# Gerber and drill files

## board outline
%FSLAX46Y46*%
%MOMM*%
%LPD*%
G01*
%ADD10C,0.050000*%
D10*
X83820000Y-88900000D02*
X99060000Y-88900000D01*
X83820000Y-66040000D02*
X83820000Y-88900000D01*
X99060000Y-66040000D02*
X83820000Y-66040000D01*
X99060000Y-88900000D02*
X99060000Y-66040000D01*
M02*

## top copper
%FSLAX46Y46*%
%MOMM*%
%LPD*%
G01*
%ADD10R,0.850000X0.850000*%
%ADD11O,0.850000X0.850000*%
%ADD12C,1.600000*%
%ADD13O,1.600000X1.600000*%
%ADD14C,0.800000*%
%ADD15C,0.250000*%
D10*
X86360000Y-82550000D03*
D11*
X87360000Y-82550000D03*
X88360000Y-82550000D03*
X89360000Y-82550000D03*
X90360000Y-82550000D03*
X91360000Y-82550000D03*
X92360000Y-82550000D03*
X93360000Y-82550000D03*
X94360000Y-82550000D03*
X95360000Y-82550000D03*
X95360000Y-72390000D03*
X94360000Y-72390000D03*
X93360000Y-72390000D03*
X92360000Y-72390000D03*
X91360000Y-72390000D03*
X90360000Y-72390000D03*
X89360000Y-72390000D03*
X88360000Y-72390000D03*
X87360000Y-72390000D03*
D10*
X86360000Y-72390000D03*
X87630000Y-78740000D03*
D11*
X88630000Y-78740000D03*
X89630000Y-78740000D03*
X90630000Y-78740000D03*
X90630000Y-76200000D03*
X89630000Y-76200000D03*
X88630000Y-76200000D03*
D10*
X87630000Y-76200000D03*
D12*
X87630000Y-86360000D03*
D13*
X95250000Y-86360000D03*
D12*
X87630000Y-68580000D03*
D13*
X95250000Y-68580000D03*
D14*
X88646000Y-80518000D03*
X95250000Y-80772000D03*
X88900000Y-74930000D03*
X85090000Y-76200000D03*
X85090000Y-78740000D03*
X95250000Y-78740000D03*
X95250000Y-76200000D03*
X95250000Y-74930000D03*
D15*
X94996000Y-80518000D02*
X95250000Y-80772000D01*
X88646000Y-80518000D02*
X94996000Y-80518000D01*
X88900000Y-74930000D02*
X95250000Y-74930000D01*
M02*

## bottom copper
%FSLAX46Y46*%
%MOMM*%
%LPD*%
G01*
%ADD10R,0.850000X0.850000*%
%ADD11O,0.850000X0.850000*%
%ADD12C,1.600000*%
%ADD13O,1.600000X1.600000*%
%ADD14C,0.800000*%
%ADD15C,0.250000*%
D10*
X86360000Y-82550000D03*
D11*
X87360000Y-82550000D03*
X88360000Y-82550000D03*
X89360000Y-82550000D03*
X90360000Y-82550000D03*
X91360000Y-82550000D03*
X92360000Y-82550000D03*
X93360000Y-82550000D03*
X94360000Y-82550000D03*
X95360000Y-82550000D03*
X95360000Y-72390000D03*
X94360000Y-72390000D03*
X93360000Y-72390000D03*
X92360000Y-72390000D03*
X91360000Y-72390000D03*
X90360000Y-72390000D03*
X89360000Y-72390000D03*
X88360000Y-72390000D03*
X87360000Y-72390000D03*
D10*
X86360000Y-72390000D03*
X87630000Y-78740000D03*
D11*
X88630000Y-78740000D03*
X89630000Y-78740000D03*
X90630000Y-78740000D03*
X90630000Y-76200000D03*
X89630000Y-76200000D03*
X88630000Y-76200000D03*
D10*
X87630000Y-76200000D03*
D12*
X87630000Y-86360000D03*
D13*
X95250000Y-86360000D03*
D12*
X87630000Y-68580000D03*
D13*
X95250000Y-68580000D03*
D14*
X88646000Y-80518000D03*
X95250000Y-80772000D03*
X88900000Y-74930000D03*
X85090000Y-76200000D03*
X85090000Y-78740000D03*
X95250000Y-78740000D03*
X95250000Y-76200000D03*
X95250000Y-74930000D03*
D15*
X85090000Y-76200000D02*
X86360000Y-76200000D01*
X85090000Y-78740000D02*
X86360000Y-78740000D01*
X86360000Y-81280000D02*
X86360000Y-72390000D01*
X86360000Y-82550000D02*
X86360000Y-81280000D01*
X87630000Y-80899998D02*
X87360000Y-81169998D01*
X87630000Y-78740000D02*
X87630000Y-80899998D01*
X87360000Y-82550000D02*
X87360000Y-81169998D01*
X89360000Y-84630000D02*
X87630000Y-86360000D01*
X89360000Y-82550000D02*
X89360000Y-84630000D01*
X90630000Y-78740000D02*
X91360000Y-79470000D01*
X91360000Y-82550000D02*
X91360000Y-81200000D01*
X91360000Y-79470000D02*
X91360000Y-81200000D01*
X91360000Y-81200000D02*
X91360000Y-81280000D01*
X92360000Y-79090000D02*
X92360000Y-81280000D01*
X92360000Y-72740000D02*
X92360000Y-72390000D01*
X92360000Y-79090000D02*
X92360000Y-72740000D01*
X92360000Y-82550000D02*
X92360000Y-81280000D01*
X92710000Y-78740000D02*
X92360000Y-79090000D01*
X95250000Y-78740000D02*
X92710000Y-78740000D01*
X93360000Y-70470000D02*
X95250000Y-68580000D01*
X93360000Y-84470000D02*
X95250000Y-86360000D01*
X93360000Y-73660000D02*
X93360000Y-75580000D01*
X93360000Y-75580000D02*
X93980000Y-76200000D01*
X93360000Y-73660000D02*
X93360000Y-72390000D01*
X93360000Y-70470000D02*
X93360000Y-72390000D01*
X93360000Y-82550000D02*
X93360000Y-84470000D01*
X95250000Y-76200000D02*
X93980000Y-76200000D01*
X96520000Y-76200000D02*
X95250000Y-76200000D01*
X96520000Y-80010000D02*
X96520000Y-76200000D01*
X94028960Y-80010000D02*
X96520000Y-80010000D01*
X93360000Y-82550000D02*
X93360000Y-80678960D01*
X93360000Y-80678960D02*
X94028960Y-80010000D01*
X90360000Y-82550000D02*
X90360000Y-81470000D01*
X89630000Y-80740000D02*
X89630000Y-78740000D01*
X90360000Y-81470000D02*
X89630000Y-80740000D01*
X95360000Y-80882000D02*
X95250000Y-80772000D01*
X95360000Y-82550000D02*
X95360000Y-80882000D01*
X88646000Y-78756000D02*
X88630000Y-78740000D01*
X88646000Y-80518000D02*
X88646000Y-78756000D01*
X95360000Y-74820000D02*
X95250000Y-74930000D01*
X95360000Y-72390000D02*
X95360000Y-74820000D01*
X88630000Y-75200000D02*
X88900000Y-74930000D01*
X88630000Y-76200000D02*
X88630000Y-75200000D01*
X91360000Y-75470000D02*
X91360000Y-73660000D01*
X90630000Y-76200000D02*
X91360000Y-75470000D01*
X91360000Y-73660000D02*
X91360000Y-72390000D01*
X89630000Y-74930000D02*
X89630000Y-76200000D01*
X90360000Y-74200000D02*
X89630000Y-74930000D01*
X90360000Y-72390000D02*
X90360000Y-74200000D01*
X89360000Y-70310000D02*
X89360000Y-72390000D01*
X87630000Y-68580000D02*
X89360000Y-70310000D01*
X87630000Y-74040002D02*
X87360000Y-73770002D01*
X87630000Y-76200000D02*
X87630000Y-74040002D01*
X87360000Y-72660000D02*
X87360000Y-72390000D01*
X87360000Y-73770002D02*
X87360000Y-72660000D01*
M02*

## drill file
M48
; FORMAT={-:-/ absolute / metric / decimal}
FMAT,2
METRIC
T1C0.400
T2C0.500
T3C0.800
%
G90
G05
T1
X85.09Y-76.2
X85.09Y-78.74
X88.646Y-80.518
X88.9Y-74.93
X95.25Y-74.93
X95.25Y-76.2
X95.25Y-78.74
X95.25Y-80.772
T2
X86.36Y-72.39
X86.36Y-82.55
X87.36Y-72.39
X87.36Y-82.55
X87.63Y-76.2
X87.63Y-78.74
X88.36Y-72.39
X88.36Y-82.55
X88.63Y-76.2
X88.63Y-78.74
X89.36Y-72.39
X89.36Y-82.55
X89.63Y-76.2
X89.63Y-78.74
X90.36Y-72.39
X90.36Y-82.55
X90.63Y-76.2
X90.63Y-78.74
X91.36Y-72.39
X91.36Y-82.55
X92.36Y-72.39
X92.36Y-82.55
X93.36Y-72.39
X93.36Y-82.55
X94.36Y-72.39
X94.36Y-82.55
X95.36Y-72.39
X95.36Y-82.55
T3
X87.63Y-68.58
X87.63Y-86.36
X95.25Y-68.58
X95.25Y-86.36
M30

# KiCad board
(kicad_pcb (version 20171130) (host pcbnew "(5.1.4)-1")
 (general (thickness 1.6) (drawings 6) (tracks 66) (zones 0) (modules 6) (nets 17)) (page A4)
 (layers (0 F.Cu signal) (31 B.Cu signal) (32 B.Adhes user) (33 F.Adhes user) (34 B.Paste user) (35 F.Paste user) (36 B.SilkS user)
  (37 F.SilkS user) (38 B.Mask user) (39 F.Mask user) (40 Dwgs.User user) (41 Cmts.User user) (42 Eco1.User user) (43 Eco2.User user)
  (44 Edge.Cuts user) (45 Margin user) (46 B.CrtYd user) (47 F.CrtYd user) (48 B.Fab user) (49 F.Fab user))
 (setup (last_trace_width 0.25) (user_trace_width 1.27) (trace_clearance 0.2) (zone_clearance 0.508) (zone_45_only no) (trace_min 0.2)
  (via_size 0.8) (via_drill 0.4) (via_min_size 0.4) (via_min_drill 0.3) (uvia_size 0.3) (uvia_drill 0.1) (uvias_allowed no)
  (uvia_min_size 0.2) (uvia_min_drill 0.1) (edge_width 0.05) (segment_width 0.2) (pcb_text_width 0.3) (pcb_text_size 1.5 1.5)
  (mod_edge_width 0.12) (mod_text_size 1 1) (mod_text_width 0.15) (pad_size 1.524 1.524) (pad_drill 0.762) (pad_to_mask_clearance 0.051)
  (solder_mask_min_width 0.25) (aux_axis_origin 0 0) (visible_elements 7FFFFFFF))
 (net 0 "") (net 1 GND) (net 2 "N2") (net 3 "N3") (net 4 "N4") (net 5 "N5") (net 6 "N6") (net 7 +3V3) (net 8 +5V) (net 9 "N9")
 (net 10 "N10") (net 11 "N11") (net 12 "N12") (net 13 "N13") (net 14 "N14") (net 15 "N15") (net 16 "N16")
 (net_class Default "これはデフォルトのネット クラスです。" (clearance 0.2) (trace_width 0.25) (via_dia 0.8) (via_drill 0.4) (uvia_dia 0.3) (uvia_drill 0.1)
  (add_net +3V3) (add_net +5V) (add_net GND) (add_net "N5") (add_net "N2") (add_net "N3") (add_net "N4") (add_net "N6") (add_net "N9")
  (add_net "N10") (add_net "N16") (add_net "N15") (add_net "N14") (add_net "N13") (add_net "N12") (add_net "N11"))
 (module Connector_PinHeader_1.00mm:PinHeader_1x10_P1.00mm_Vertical (layer F.Cu) (at 86.36 82.55 90)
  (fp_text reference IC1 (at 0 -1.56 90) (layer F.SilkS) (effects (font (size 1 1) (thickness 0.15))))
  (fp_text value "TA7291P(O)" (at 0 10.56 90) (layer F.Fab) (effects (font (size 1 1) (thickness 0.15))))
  (pad 1 thru_hole rect (at 0 0 90) (size 0.85 0.85) (drill 0.5) (layers *.Cu *.Mask) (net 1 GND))
  (pad 2 thru_hole oval (at 0 1 90) (size 0.85 0.85) (drill 0.5) (layers *.Cu *.Mask) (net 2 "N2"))
  (pad 3 thru_hole oval (at 0 2 90) (size 0.85 0.85) (drill 0.5) (layers *.Cu *.Mask) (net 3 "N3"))
  (pad 4 thru_hole oval (at 0 3 90) (size 0.85 0.85) (drill 0.5) (layers *.Cu *.Mask) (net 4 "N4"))
  (pad 5 thru_hole oval (at 0 4 90) (size 0.85 0.85) (drill 0.5) (layers *.Cu *.Mask) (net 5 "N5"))
  (pad 6 thru_hole oval (at 0 5 90) (size 0.85 0.85) (drill 0.5) (layers *.Cu *.Mask) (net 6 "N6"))
  (pad 7 thru_hole oval (at 0 6 90) (size 0.85 0.85) (drill 0.5) (layers *.Cu *.Mask) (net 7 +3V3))
  (pad 8 thru_hole oval (at 0 7 90) (size 0.85 0.85) (drill 0.5) (layers *.Cu *.Mask) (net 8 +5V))
  (pad 9 thru_hole oval (at 0 8 90) (size 0.85 0.85) (drill 0.5) (layers *.Cu *.Mask) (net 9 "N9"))
  (pad 10 thru_hole oval (at 0 9 90) (size 0.85 0.85) (drill 0.5) (layers *.Cu *.Mask) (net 5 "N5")))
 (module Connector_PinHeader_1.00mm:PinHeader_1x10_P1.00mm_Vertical (layer F.Cu) (at 86.36 72.39 90)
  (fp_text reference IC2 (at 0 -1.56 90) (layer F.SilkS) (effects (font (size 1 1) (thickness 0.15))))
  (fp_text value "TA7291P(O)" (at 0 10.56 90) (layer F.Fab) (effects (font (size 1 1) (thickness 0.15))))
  (pad 10 thru_hole oval (at 0 9 90) (size 0.85 0.85) (drill 0.5) (layers *.Cu *.Mask) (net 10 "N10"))
  (pad 9 thru_hole oval (at 0 8 90) (size 0.85 0.85) (drill 0.5) (layers *.Cu *.Mask) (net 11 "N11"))
  (pad 8 thru_hole oval (at 0 7 90) (size 0.85 0.85) (drill 0.5) (layers *.Cu *.Mask) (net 8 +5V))
  (pad 7 thru_hole oval (at 0 6 90) (size 0.85 0.85) (drill 0.5) (layers *.Cu *.Mask) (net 7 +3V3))
  (pad 6 thru_hole oval (at 0 5 90) (size 0.85 0.85) (drill 0.5) (layers *.Cu *.Mask) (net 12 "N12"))
  (pad 5 thru_hole oval (at 0 4 90) (size 0.85 0.85) (drill 0.5) (layers *.Cu *.Mask) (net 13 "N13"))
  (pad 4 thru_hole oval (at 0 3 90) (size 0.85 0.85) (drill 0.5) (layers *.Cu *.Mask) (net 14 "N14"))
  (pad 3 thru_hole oval (at 0 2 90) (size 0.85 0.85) (drill 0.5) (layers *.Cu *.Mask) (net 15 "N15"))
  (pad 2 thru_hole oval (at 0 1 90) (size 0.85 0.85) (drill 0.5) (layers *.Cu *.Mask) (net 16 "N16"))
  (pad 1 thru_hole rect (at 0 0 90) (size 0.85 0.85) (drill 0.5) (layers *.Cu *.Mask) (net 1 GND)))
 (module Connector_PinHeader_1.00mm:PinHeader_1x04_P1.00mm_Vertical (layer F.Cu) (at 87.63 78.74 90)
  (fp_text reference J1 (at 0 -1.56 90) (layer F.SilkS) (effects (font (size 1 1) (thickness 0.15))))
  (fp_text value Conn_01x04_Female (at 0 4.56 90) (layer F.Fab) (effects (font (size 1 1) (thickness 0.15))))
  (pad 1 thru_hole rect (at 0 0 90) (size 0.85 0.85) (drill 0.5) (layers *.Cu *.Mask) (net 2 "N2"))
  (pad 2 thru_hole oval (at 0 1 90) (size 0.85 0.85) (drill 0.5) (layers *.Cu *.Mask) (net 5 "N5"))
  (pad 3 thru_hole oval (at 0 2 90) (size 0.85 0.85) (drill 0.5) (layers *.Cu *.Mask) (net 5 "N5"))
  (pad 4 thru_hole oval (at 0 3 90) (size 0.85 0.85) (drill 0.5) (layers *.Cu *.Mask) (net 6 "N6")))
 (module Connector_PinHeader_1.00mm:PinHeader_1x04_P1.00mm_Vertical (layer F.Cu) (at 87.63 76.2 90)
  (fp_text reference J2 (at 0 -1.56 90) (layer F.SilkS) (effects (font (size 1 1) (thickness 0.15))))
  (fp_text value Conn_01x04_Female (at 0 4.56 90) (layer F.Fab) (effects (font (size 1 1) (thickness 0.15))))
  (pad 4 thru_hole oval (at 0 3 90) (size 0.85 0.85) (drill 0.5) (layers *.Cu *.Mask) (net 12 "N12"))
  (pad 3 thru_hole oval (at 0 2 90) (size 0.85 0.85) (drill 0.5) (layers *.Cu *.Mask) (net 13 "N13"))
  (pad 2 thru_hole oval (at 0 1 90) (size 0.85 0.85) (drill 0.5) (layers *.Cu *.Mask) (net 10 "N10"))
  (pad 1 thru_hole rect (at 0 0 90) (size 0.85 0.85) (drill 0.5) (layers *.Cu *.Mask) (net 16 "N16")))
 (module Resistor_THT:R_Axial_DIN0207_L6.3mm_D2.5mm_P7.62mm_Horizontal (layer F.Cu) (at 87.63 86.36)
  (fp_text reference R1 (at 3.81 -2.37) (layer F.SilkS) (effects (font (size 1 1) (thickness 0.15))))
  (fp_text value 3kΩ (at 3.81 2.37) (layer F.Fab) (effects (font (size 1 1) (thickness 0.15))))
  (pad 1 thru_hole circle (at 0 0) (size 1.6 1.6) (drill 0.8) (layers *.Cu *.Mask) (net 4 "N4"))
  (pad 2 thru_hole oval (at 7.62 0) (size 1.6 1.6) (drill 0.8) (layers *.Cu *.Mask) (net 8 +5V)))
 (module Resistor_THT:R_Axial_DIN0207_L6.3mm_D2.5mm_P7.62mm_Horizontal (layer F.Cu) (at 87.63 68.58)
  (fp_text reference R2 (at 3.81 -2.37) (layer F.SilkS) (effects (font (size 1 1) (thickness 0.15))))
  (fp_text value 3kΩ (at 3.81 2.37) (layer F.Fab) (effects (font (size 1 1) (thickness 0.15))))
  (pad 1 thru_hole circle (at 0 0) (size 1.6 1.6) (drill 0.8) (layers *.Cu *.Mask) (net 14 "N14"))
  (pad 2 thru_hole oval (at 7.62 0) (size 1.6 1.6) (drill 0.8) (layers *.Cu *.Mask) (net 8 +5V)))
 (gr_line (start 83.82 88.9) (end 99.06 88.9) (layer Edge.Cuts) (width 0.05))
 (gr_line (start 83.82 66.04) (end 83.82 88.9) (layer Edge.Cuts) (width 0.05))
 (gr_line (start 99.06 66.04) (end 83.82 66.04) (layer Edge.Cuts) (width 0.05))
 (gr_line (start 99.06 88.9) (end 99.06 66.04) (layer Edge.Cuts) (width 0.05))
 (via (at 88.646 80.518) (size 0.8) (drill 0.4) (layers F.Cu B.Cu) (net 5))
 (via (at 95.25 80.772) (size 0.8) (drill 0.4) (layers F.Cu B.Cu) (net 5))
 (segment (start 94.996 80.518) (end 95.25 80.772) (width 0.25) (layer F.Cu) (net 5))
 (segment (start 88.646 80.518) (end 94.996 80.518) (width 0.25) (layer F.Cu) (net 5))
 (via (at 88.9 74.93) (size 0.8) (drill 0.4) (layers F.Cu B.Cu) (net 10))
 (via (at 85.09 76.2) (size 0.8) (drill 0.4) (layers F.Cu B.Cu) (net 1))
 (via (at 85.09 78.74) (size 0.8) (drill 0.4) (layers F.Cu B.Cu) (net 1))
 (segment (start 85.09 76.2) (end 86.36 76.2) (width 0.25) (layer B.Cu) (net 1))
 (segment (start 85.09 78.74) (end 86.36 78.74) (width 0.25) (layer B.Cu) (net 1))
 (segment (start 86.36 81.28) (end 86.36 72.39) (width 0.25) (layer B.Cu) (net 1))
 (segment (start 86.36 82.55) (end 86.36 81.28) (width 0.25) (layer B.Cu) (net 1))
 (segment (start 87.63 80.899998) (end 87.36 81.169998) (width 0.25) (layer B.Cu) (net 2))
 (segment (start 87.63 78.74) (end 87.63 80.899998) (width 0.25) (layer B.Cu) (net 2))
 (segment (start 87.36 82.55) (end 87.36 81.169998) (width 0.25) (layer B.Cu) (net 2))
 (segment (start 89.36 84.63) (end 87.63 86.36) (width 0.25) (layer B.Cu) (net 4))
 (segment (start 89.36 82.55) (end 89.36 84.63) (width 0.25) (layer B.Cu) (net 4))
 (segment (start 90.63 78.74) (end 91.36 79.47) (width 0.25) (layer B.Cu) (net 6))
 (segment (start 91.36 82.55) (end 91.36 81.2) (width 0.25) (layer B.Cu) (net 6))
 (segment (start 91.36 79.47) (end 91.36 81.2) (width 0.25) (layer B.Cu) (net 6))
 (segment (start 91.36 81.2) (end 91.36 81.28) (width 0.25) (layer B.Cu) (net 6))
 (via (at 95.25 78.74) (size 0.8) (drill 0.4) (layers F.Cu B.Cu) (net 7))
 (segment (start 92.36 79.09) (end 92.36 81.28) (width 0.25) (layer B.Cu) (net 7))
 (segment (start 92.36 72.74) (end 92.36 72.39) (width 0.25) (layer B.Cu) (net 7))
 (segment (start 92.36 79.09) (end 92.36 72.74) (width 0.25) (layer B.Cu) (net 7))
 (segment (start 92.36 82.55) (end 92.36 81.28) (width 0.25) (layer B.Cu) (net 7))
 (segment (start 92.71 78.74) (end 92.36 79.09) (width 0.25) (layer B.Cu) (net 7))
 (segment (start 95.25 78.74) (end 92.71 78.74) (width 0.25) (layer B.Cu) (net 7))
 (via (at 95.25 76.2) (size 0.8) (drill 0.4) (layers F.Cu B.Cu) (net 8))
 (segment (start 93.36 70.47) (end 95.25 68.58) (width 0.25) (layer B.Cu) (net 8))
 (segment (start 93.36 84.47) (end 95.25 86.36) (width 0.25) (layer B.Cu) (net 8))
 (segment (start 93.36 73.66) (end 93.36 75.58) (width 0.25) (layer B.Cu) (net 8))
 (segment (start 93.36 75.58) (end 93.98 76.2) (width 0.25) (layer B.Cu) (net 8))
 (segment (start 93.36 73.66) (end 93.36 72.39) (width 0.25) (layer B.Cu) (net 8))
 (segment (start 93.36 70.47) (end 93.36 72.39) (width 0.25) (layer B.Cu) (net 8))
 (segment (start 93.36 82.55) (end 93.36 84.47) (width 0.25) (layer B.Cu) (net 8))
 (segment (start 95.25 76.2) (end 93.98 76.2) (width 0.25) (layer B.Cu) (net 8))
 (segment (start 96.52 76.2) (end 95.25 76.2) (width 0.25) (layer B.Cu) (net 8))
 (segment (start 96.52 80.01) (end 96.52 76.2) (width 0.25) (layer B.Cu) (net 8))
 (segment (start 94.02896 80.01) (end 96.52 80.01) (width 0.25) (layer B.Cu) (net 8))
 (segment (start 93.36 82.55) (end 93.36 80.67896) (width 0.25) (layer B.Cu) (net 8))
 (segment (start 93.36 80.67896) (end 94.02896 80.01) (width 0.25) (layer B.Cu) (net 8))
 (segment (start 90.36 82.55) (end 90.36 81.47) (width 0.25) (layer B.Cu) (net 5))
 (segment (start 89.63 80.74) (end 89.63 78.74) (width 0.25) (layer B.Cu) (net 5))
 (segment (start 90.36 81.47) (end 89.63 80.74) (width 0.25) (layer B.Cu) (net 5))
 (segment (start 95.36 80.882) (end 95.25 80.772) (width 0.25) (layer B.Cu) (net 5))
 (segment (start 95.36 82.55) (end 95.36 80.882) (width 0.25) (layer B.Cu) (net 5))
 (segment (start 88.646 78.756) (end 88.63 78.74) (width 0.25) (layer B.Cu) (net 5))
 (segment (start 88.646 80.518) (end 88.646 78.756) (width 0.25) (layer B.Cu) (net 5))
 (via (at 95.25 74.93) (size 0.8) (drill 0.4) (layers F.Cu B.Cu) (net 10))
 (segment (start 95.36 74.82) (end 95.25 74.93) (width 0.25) (layer B.Cu) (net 10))
 (segment (start 95.36 72.39) (end 95.36 74.82) (width 0.25) (layer B.Cu) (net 10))
 (segment (start 88.63 75.2) (end 88.9 74.93) (width 0.25) (layer B.Cu) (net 10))
 (segment (start 88.63 76.2) (end 88.63 75.2) (width 0.25) (layer B.Cu) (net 10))
 (segment (start 88.9 74.93) (end 95.25 74.93) (width 0.25) (layer F.Cu) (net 10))
 (segment (start 91.36 75.47) (end 91.36 73.66) (width 0.25) (layer B.Cu) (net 12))
 (segment (start 90.63 76.2) (end 91.36 75.47) (width 0.25) (layer B.Cu) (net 12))
 (segment (start 91.36 73.66) (end 91.36 72.39) (width 0.25) (layer B.Cu) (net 12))
 (segment (start 89.63 74.93) (end 89.63 76.2) (width 0.25) (layer B.Cu) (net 13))
 (segment (start 90.36 74.2) (end 89.63 74.93) (width 0.25) (layer B.Cu) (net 13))
 (segment (start 90.36 72.39) (end 90.36 74.2) (width 0.25) (layer B.Cu) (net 13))
 (segment (start 89.36 70.31) (end 89.36 72.39) (width 0.25) (layer B.Cu) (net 14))
 (segment (start 87.63 68.58) (end 89.36 70.31) (width 0.25) (layer B.Cu) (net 14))
 (segment (start 87.63 74.040002) (end 87.36 73.770002) (width 0.25) (layer B.Cu) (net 16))
 (segment (start 87.63 76.2) (end 87.63 74.040002) (width 0.25) (layer B.Cu) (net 16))
 (segment (start 87.36 72.66) (end 87.36 72.39) (width 0.25) (layer B.Cu) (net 16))
 (segment (start 87.36 73.770002) (end 87.36 72.66) (width 0.25) (layer B.Cu) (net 16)))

